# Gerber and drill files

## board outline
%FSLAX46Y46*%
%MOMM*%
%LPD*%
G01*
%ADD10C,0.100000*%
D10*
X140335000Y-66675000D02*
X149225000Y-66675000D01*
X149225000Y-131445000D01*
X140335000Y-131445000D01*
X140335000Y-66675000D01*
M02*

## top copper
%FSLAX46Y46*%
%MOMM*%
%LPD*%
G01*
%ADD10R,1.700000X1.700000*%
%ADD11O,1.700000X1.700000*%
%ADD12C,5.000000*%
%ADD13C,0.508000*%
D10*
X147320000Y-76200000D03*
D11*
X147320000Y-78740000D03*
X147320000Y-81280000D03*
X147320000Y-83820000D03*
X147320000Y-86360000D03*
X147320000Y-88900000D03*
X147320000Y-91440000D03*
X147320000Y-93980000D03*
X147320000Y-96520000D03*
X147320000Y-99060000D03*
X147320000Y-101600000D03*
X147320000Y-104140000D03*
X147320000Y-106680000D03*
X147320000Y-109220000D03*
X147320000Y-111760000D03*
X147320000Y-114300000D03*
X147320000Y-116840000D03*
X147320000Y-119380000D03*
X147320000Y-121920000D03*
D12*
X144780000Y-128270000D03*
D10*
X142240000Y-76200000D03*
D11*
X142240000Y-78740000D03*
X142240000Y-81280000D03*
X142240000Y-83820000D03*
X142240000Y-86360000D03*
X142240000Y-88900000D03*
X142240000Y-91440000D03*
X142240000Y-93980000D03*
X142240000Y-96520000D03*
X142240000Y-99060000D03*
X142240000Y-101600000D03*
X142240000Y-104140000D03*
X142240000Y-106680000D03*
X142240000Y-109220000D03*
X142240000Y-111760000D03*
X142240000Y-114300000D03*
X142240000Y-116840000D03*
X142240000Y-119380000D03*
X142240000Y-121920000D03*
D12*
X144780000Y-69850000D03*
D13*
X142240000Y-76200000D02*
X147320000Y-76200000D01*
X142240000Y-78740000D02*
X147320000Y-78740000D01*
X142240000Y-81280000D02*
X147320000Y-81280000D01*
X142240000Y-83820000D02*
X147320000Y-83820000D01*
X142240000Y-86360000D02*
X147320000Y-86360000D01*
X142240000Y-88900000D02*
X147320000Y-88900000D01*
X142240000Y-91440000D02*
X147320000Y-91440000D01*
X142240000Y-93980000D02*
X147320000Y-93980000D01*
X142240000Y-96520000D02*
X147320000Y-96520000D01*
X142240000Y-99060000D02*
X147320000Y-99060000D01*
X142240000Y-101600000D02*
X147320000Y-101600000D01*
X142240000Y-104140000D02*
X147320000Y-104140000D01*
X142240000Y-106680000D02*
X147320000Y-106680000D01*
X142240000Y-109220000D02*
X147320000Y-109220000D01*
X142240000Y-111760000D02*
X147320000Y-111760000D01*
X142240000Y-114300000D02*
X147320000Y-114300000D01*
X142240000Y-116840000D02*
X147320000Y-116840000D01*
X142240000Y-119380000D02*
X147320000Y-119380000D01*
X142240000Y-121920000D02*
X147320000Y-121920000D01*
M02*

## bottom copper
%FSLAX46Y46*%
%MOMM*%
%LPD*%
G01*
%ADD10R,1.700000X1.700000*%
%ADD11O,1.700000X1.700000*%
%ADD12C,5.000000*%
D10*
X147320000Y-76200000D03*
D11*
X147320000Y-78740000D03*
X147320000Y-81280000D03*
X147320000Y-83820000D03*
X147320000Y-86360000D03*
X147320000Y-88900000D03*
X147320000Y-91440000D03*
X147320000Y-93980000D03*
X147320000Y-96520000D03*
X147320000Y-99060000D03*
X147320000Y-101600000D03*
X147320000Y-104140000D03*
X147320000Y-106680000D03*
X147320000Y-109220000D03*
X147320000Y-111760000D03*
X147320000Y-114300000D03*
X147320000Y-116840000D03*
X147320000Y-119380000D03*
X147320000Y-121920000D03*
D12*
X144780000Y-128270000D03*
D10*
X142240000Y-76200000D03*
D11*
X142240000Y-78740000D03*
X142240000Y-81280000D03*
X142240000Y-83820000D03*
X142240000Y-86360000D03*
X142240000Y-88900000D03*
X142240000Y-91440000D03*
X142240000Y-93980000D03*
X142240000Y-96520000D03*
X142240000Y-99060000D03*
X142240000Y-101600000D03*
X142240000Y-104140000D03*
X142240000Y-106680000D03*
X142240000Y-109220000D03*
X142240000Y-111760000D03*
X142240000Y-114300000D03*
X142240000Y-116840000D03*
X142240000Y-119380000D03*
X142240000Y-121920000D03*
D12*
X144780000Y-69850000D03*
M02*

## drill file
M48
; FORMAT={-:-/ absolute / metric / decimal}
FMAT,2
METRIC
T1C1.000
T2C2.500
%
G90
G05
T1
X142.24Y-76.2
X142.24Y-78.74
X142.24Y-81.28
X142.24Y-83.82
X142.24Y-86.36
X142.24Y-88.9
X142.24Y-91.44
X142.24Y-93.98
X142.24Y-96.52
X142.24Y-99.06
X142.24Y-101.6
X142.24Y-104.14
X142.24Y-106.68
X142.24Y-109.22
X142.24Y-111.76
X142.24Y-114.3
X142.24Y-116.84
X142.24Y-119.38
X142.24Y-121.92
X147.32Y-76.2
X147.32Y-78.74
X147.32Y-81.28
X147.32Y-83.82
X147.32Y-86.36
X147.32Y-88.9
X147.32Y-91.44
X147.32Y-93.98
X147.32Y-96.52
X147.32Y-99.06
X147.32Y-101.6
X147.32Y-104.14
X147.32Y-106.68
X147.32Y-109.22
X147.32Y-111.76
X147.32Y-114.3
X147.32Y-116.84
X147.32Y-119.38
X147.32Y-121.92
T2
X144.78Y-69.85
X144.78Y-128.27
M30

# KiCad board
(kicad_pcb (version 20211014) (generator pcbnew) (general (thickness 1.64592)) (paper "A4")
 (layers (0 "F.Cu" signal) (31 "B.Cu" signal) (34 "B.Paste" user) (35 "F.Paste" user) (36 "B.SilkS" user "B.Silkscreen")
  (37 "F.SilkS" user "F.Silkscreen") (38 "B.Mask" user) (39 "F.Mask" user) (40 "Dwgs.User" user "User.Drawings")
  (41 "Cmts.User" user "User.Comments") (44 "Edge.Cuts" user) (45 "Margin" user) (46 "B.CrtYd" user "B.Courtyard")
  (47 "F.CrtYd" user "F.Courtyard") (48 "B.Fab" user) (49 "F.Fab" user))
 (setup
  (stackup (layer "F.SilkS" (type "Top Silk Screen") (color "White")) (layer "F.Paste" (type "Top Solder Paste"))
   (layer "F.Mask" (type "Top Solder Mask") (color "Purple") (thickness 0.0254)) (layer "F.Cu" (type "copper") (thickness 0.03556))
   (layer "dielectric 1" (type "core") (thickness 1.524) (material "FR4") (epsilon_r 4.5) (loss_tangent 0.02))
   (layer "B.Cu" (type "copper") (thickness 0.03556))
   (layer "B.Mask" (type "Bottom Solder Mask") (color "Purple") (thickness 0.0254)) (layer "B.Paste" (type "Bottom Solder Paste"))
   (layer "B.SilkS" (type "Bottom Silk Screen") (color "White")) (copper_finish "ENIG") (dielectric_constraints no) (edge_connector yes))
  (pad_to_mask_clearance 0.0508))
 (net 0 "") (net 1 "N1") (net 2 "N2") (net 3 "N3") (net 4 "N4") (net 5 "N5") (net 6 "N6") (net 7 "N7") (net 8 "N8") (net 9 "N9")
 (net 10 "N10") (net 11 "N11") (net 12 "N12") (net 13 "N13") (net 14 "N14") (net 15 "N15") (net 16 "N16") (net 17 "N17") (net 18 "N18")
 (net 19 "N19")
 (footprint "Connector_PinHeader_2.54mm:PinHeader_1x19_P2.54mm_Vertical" (layer "F.Cu") (at 147.32 76.2)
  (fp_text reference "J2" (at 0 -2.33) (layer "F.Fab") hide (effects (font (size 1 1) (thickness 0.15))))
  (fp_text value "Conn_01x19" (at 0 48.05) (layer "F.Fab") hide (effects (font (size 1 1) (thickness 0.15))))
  (pad "1" thru_hole rect (at 0 0) (size 1.7 1.7) (drill 1) (layers *.Cu *.Mask) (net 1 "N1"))
  (pad "2" thru_hole oval (at 0 2.54) (size 1.7 1.7) (drill 1) (layers *.Cu *.Mask) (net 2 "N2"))
  (pad "3" thru_hole oval (at 0 5.08) (size 1.7 1.7) (drill 1) (layers *.Cu *.Mask) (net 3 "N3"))
  (pad "4" thru_hole oval (at 0 7.62) (size 1.7 1.7) (drill 1) (layers *.Cu *.Mask) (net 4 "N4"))
  (pad "5" thru_hole oval (at 0 10.16) (size 1.7 1.7) (drill 1) (layers *.Cu *.Mask) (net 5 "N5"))
  (pad "6" thru_hole oval (at 0 12.7) (size 1.7 1.7) (drill 1) (layers *.Cu *.Mask) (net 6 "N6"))
  (pad "7" thru_hole oval (at 0 15.24) (size 1.7 1.7) (drill 1) (layers *.Cu *.Mask) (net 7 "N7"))
  (pad "8" thru_hole oval (at 0 17.78) (size 1.7 1.7) (drill 1) (layers *.Cu *.Mask) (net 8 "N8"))
  (pad "9" thru_hole oval (at 0 20.32) (size 1.7 1.7) (drill 1) (layers *.Cu *.Mask) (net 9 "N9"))
  (pad "10" thru_hole oval (at 0 22.86) (size 1.7 1.7) (drill 1) (layers *.Cu *.Mask) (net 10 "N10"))
  (pad "11" thru_hole oval (at 0 25.4) (size 1.7 1.7) (drill 1) (layers *.Cu *.Mask) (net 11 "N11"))
  (pad "12" thru_hole oval (at 0 27.94) (size 1.7 1.7) (drill 1) (layers *.Cu *.Mask) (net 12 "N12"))
  (pad "13" thru_hole oval (at 0 30.48) (size 1.7 1.7) (drill 1) (layers *.Cu *.Mask) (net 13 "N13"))
  (pad "14" thru_hole oval (at 0 33.02) (size 1.7 1.7) (drill 1) (layers *.Cu *.Mask) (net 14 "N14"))
  (pad "15" thru_hole oval (at 0 35.56) (size 1.7 1.7) (drill 1) (layers *.Cu *.Mask) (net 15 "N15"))
  (pad "16" thru_hole oval (at 0 38.1) (size 1.7 1.7) (drill 1) (layers *.Cu *.Mask) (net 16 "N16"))
  (pad "17" thru_hole oval (at 0 40.64) (size 1.7 1.7) (drill 1) (layers *.Cu *.Mask) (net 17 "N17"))
  (pad "18" thru_hole oval (at 0 43.18) (size 1.7 1.7) (drill 1) (layers *.Cu *.Mask) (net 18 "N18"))
  (pad "19" thru_hole oval (at 0 45.72) (size 1.7 1.7) (drill 1) (layers *.Cu *.Mask) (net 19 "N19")))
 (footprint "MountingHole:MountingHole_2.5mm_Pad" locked (layer "F.Cu") (at 144.78 128.27)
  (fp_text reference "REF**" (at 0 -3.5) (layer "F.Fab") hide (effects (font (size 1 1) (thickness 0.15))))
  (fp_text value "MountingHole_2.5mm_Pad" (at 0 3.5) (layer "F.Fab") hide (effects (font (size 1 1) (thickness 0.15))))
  (pad "1" thru_hole circle locked (at 0 0) (size 5 5) (drill 2.5) (layers *.Cu *.Mask)))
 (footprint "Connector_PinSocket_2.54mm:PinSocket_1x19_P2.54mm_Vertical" (layer "F.Cu") (at 142.24 76.2)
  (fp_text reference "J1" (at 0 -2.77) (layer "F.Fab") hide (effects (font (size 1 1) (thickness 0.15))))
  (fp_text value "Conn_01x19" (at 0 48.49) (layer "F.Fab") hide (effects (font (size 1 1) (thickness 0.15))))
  (pad "1" thru_hole rect (at 0 0) (size 1.7 1.7) (drill 1) (layers *.Cu *.Mask) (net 1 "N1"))
  (pad "2" thru_hole oval (at 0 2.54) (size 1.7 1.7) (drill 1) (layers *.Cu *.Mask) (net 2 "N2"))
  (pad "3" thru_hole oval (at 0 5.08) (size 1.7 1.7) (drill 1) (layers *.Cu *.Mask) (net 3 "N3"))
  (pad "4" thru_hole oval (at 0 7.62) (size 1.7 1.7) (drill 1) (layers *.Cu *.Mask) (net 4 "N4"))
  (pad "5" thru_hole oval (at 0 10.16) (size 1.7 1.7) (drill 1) (layers *.Cu *.Mask) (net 5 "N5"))
  (pad "6" thru_hole oval (at 0 12.7) (size 1.7 1.7) (drill 1) (layers *.Cu *.Mask) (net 6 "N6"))
  (pad "7" thru_hole oval (at 0 15.24) (size 1.7 1.7) (drill 1) (layers *.Cu *.Mask) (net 7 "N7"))
  (pad "8" thru_hole oval (at 0 17.78) (size 1.7 1.7) (drill 1) (layers *.Cu *.Mask) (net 8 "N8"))
  (pad "9" thru_hole oval (at 0 20.32) (size 1.7 1.7) (drill 1) (layers *.Cu *.Mask) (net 9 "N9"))
  (pad "10" thru_hole oval (at 0 22.86) (size 1.7 1.7) (drill 1) (layers *.Cu *.Mask) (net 10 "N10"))
  (pad "11" thru_hole oval (at 0 25.4) (size 1.7 1.7) (drill 1) (layers *.Cu *.Mask) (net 11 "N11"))
  (pad "12" thru_hole oval (at 0 27.94) (size 1.7 1.7) (drill 1) (layers *.Cu *.Mask) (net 12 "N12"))
  (pad "13" thru_hole oval (at 0 30.48) (size 1.7 1.7) (drill 1) (layers *.Cu *.Mask) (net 13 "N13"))
  (pad "14" thru_hole oval (at 0 33.02) (size 1.7 1.7) (drill 1) (layers *.Cu *.Mask) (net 14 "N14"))
  (pad "15" thru_hole oval (at 0 35.56) (size 1.7 1.7) (drill 1) (layers *.Cu *.Mask) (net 15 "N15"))
  (pad "16" thru_hole oval (at 0 38.1) (size 1.7 1.7) (drill 1) (layers *.Cu *.Mask) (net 16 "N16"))
  (pad "17" thru_hole oval (at 0 40.64) (size 1.7 1.7) (drill 1) (layers *.Cu *.Mask) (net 17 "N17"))
  (pad "18" thru_hole oval (at 0 43.18) (size 1.7 1.7) (drill 1) (layers *.Cu *.Mask) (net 18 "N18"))
  (pad "19" thru_hole oval (at 0 45.72) (size 1.7 1.7) (drill 1) (layers *.Cu *.Mask) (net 19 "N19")))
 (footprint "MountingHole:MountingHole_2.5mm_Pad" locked (layer "F.Cu") (at 144.78 69.85)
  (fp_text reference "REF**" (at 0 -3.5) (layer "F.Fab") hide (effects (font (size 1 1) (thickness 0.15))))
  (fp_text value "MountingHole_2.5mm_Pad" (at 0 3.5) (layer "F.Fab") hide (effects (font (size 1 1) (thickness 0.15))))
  (pad "1" thru_hole circle locked (at 0 0) (size 5 5) (drill 2.5) (layers *.Cu *.Mask)))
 (gr_rect (start 140.335 66.675) (end 149.225 131.445) (layer "Edge.Cuts") (width 0.1) (fill none))
 (segment (start 142.24 76.2) (end 147.32 76.2) (width 0.508) (layer "F.Cu") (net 1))
 (segment (start 142.24 78.74) (end 147.32 78.74) (width 0.508) (layer "F.Cu") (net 2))
 (segment (start 142.24 81.28) (end 147.32 81.28) (width 0.508) (layer "F.Cu") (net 3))
 (segment (start 142.24 83.82) (end 147.32 83.82) (width 0.508) (layer "F.Cu") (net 4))
 (segment (start 142.24 86.36) (end 147.32 86.36) (width 0.508) (layer "F.Cu") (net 5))
 (segment (start 142.24 88.9) (end 147.32 88.9) (width 0.508) (layer "F.Cu") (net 6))
 (segment (start 142.24 91.44) (end 147.32 91.44) (width 0.508) (layer "F.Cu") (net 7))
 (segment (start 142.24 93.98) (end 147.32 93.98) (width 0.508) (layer "F.Cu") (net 8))
 (segment (start 142.24 96.52) (end 147.32 96.52) (width 0.508) (layer "F.Cu") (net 9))
 (segment (start 142.24 99.06) (end 147.32 99.06) (width 0.508) (layer "F.Cu") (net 10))
 (segment (start 142.24 101.6) (end 147.32 101.6) (width 0.508) (layer "F.Cu") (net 11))
 (segment (start 142.24 104.14) (end 147.32 104.14) (width 0.508) (layer "F.Cu") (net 12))
 (segment (start 142.24 106.68) (end 147.32 106.68) (width 0.508) (layer "F.Cu") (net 13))
 (segment (start 142.24 109.22) (end 147.32 109.22) (width 0.508) (layer "F.Cu") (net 14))
 (segment (start 142.24 111.76) (end 147.32 111.76) (width 0.508) (layer "F.Cu") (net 15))
 (segment (start 142.24 114.3) (end 147.32 114.3) (width 0.508) (layer "F.Cu") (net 16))
 (segment (start 142.24 116.84) (end 147.32 116.84) (width 0.508) (layer "F.Cu") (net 17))
 (segment (start 142.24 119.38) (end 147.32 119.38) (width 0.508) (layer "F.Cu") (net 18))
 (segment (start 142.24 121.92) (end 147.32 121.92) (width 0.508) (layer "F.Cu") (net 19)))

